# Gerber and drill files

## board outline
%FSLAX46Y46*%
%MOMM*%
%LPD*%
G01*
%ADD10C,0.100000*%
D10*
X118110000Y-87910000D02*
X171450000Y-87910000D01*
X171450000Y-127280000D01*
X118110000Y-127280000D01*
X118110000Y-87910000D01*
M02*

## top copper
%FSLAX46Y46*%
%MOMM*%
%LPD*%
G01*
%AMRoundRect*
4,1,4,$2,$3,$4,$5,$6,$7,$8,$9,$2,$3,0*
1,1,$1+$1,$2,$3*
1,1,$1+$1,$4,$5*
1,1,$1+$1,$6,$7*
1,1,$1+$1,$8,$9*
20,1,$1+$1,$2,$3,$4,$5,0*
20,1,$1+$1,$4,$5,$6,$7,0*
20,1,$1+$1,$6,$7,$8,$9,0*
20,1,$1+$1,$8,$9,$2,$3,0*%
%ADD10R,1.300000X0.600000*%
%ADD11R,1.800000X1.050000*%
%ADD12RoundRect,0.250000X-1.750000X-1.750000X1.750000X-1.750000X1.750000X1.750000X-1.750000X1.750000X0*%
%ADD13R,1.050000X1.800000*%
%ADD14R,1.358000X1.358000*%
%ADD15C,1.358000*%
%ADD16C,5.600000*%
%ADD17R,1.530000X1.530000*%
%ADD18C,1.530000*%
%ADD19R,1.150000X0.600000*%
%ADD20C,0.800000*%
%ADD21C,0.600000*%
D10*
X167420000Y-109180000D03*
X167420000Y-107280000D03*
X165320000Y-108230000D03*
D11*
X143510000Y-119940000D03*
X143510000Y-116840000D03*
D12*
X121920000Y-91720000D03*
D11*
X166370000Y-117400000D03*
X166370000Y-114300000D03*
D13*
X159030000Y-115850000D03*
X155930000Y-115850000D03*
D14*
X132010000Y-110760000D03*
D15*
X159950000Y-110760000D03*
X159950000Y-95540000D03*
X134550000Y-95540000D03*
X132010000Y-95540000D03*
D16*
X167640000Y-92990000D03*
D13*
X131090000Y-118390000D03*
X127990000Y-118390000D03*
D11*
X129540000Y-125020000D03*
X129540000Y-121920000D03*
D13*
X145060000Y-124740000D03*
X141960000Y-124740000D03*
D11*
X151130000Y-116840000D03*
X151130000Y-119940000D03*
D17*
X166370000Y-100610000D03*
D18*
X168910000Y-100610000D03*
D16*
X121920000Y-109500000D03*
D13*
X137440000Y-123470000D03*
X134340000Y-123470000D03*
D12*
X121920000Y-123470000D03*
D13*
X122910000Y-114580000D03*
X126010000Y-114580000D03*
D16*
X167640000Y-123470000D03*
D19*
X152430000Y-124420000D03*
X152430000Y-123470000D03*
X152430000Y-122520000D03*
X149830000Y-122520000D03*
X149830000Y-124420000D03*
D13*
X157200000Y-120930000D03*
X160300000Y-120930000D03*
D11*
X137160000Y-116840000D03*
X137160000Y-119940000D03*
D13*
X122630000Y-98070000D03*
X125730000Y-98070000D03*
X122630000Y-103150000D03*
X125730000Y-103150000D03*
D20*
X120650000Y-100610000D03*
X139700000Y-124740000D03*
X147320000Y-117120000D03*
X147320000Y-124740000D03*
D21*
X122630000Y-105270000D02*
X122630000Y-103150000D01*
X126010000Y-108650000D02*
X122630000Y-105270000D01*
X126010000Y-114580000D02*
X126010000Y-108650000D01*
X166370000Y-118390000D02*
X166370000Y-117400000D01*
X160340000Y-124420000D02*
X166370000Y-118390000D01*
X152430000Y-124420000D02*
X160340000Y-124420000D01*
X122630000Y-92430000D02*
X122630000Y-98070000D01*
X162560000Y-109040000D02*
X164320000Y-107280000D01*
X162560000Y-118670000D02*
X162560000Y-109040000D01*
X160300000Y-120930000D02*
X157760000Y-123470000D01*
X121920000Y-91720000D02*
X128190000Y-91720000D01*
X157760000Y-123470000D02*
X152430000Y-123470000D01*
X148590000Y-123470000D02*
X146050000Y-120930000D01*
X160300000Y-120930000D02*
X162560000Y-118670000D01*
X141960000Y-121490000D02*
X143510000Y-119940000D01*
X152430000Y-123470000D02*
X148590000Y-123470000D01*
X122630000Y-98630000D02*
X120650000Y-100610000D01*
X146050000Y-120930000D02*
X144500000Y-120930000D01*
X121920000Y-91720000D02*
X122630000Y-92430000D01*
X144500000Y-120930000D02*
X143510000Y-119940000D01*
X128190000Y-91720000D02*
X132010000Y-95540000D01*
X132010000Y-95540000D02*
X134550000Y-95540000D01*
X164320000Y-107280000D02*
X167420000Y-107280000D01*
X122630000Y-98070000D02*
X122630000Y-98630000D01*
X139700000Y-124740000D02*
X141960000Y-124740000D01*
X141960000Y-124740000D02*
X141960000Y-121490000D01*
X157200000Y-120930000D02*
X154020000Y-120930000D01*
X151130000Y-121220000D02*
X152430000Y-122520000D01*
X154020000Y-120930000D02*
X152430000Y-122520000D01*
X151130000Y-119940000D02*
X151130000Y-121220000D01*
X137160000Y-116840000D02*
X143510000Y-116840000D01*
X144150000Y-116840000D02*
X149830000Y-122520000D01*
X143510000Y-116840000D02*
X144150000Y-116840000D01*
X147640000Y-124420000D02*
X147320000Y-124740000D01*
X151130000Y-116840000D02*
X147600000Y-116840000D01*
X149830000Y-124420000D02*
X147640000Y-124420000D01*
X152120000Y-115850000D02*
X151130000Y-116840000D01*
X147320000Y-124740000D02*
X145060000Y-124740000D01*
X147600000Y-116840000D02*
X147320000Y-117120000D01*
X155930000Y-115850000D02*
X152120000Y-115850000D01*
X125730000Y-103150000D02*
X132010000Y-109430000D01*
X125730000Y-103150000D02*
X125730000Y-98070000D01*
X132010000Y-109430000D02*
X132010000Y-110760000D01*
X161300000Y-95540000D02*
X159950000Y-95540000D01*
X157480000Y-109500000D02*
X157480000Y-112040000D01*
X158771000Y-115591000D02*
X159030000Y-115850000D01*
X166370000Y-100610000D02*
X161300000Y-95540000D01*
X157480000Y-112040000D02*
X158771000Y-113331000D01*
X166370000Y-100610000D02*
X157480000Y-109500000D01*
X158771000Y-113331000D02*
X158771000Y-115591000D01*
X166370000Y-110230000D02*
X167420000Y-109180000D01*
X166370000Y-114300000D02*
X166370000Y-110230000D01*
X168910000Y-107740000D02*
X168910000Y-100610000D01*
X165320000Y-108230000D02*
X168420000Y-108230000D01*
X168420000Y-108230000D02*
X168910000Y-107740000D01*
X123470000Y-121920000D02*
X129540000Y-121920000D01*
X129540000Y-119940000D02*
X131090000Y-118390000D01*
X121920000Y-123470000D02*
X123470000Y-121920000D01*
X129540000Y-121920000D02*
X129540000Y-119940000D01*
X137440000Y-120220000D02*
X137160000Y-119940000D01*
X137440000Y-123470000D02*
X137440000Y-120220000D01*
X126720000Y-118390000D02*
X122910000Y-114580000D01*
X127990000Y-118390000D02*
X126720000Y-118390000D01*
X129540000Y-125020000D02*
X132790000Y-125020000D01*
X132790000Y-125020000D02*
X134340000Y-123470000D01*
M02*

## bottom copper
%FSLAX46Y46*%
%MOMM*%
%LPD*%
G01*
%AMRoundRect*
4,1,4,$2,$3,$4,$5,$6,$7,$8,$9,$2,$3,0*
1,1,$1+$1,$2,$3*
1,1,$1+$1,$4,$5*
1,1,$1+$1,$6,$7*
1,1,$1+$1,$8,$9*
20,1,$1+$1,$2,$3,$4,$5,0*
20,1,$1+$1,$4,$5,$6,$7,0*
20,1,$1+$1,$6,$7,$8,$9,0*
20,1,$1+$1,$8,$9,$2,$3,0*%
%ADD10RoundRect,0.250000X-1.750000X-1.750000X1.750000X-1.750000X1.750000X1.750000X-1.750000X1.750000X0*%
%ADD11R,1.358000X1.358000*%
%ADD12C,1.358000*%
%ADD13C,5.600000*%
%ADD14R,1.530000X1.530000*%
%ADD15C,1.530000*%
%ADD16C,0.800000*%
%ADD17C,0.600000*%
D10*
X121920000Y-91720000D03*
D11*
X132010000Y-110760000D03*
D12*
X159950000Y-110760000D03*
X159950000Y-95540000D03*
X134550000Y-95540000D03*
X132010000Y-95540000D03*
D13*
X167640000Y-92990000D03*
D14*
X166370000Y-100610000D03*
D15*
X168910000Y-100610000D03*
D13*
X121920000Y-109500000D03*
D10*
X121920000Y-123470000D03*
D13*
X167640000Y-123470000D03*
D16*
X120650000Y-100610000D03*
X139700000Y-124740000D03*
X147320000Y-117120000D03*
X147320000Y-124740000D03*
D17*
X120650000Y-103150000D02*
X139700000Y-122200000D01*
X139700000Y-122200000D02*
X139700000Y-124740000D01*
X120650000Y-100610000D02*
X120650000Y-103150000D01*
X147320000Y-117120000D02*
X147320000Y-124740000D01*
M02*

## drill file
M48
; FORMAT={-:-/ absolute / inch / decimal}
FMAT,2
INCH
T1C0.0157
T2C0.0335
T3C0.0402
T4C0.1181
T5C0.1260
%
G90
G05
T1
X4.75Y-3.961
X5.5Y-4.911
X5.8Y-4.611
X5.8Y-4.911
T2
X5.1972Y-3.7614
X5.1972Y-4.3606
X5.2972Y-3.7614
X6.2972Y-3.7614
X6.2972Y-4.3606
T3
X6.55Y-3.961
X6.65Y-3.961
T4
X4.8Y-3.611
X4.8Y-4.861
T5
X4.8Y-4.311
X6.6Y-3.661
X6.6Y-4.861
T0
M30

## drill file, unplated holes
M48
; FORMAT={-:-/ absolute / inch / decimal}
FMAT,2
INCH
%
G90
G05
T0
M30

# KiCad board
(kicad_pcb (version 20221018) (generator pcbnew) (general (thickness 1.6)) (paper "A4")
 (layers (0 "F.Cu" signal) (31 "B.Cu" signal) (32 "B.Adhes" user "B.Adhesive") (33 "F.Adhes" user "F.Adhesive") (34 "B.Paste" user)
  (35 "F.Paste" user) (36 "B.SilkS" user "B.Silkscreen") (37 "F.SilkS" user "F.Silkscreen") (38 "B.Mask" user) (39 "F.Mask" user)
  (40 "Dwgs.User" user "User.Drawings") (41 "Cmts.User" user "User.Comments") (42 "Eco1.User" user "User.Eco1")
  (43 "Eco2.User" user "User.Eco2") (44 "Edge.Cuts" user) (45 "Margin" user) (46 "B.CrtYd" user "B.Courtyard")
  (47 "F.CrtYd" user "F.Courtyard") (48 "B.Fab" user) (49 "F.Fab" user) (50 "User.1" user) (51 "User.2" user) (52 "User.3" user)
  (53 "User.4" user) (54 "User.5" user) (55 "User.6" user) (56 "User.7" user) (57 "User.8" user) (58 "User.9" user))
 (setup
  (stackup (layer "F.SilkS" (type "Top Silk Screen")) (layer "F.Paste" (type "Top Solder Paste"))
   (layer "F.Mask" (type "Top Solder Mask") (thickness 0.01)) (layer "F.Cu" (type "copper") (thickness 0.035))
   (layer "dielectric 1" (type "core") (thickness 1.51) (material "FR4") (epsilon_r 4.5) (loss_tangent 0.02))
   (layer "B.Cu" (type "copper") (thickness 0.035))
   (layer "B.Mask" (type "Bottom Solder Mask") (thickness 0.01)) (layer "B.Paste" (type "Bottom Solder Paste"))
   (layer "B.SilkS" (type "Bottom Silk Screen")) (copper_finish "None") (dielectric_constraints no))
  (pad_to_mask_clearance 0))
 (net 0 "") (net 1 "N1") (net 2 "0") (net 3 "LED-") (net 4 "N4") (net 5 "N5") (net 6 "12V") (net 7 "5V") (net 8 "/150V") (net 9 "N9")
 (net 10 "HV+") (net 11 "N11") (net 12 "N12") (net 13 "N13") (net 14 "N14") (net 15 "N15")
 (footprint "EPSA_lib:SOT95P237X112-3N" (layer "F.Cu") (at 166.37 108.23 180)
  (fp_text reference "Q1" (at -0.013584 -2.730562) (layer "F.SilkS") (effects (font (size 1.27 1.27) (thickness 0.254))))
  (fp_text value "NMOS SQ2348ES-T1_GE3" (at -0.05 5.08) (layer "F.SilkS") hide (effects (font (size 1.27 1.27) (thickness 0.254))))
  (pad "1" smd rect (at -1.05 -0.95 270) (size 0.6 1.3) (layers "F.Cu" "F.Paste" "F.Mask") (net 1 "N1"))
  (pad "2" smd rect (at -1.05 0.95 270) (size 0.6 1.3) (layers "F.Cu" "F.Paste" "F.Mask") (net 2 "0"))
  (pad "3" smd rect (at 1.05 0 270) (size 0.6 1.3) (layers "F.Cu" "F.Paste" "F.Mask") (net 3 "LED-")))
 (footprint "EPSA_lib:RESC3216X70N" (layer "F.Cu") (at 143.51 118.39 90)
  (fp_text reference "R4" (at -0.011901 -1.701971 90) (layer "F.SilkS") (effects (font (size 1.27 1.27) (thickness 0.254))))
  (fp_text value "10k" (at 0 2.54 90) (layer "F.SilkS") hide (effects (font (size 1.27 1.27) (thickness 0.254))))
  (pad "1" smd rect (at -1.55 0 90) (size 1.05 1.8) (layers "F.Cu" "F.Paste" "F.Mask") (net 2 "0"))
  (pad "2" smd rect (at 1.55 0 90) (size 1.05 1.8) (layers "F.Cu" "F.Paste" "F.Mask") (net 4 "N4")))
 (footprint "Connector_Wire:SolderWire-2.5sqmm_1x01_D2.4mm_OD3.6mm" (layer "F.Cu") (at 121.92 91.72)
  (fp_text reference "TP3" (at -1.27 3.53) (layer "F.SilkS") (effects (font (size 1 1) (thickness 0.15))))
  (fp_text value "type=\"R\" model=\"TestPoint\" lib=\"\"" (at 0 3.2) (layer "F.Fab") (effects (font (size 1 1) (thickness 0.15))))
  (pad "1" thru_hole roundrect (at 0 0) (size 4 4) (drill 3) (layers "*.Cu" "*.Mask") (roundrect_rratio 0.0625) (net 2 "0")))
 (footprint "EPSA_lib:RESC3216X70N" (layer "F.Cu") (at 166.37 115.85 90)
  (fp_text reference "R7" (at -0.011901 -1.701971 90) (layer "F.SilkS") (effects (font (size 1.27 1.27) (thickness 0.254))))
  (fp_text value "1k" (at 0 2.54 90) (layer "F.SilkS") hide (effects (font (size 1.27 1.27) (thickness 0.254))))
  (pad "1" smd rect (at -1.55 0 90) (size 1.05 1.8) (layers "F.Cu" "F.Paste" "F.Mask") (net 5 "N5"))
  (pad "2" smd rect (at 1.55 0 90) (size 1.05 1.8) (layers "F.Cu" "F.Paste" "F.Mask") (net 1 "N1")))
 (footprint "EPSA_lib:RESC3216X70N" (layer "F.Cu") (at 157.48 115.85 180)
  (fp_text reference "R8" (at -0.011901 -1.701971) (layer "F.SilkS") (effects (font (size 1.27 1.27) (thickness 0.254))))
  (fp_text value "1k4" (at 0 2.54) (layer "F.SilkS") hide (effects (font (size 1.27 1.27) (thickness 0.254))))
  (pad "1" smd rect (at -1.55 0 180) (size 1.05 1.8) (layers "F.Cu" "F.Paste" "F.Mask") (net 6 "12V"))
  (pad "2" smd rect (at 1.55 0 180) (size 1.05 1.8) (layers "F.Cu" "F.Paste" "F.Mask") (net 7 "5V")))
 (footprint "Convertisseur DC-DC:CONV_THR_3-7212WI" (layer "F.Cu") (at 146.05 103.15 180)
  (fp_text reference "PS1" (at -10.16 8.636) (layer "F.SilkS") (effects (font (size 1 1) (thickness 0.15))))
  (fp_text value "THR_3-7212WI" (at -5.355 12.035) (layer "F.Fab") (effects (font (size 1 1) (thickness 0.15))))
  (pad "1" thru_hole rect (at 14.04 -7.61 180) (size 1.358 1.358) (drill 0.85) (layers "*.Cu" "*.Mask") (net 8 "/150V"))
  (pad "12" thru_hole circle (at -13.9 -7.61 180) (size 1.358 1.358) (drill 0.85) (layers "*.Cu" "*.Mask") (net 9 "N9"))
  (pad "13" thru_hole circle (at -13.9 7.61 180) (size 1.358 1.358) (drill 0.85) (layers "*.Cu" "*.Mask") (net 6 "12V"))
  (pad "23" thru_hole circle (at 11.5 7.61 180) (size 1.358 1.358) (drill 0.85) (layers "*.Cu" "*.Mask") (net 2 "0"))
  (pad "24" thru_hole circle (at 14.04 7.61 180) (size 1.358 1.358) (drill 0.85) (layers "*.Cu" "*.Mask") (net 2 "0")))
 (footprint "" (layer "F.Cu") (at 167.64 92.99)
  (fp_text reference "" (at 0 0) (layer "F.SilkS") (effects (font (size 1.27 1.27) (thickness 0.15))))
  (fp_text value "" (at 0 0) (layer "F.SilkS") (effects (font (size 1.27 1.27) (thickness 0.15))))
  (pad "1" thru_hole circle (at 0 0) (size 5.6 5.6) (drill 3.2) (layers "*.Cu" "*.Mask")))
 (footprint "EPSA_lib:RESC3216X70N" (layer "F.Cu") (at 129.54 118.39 180)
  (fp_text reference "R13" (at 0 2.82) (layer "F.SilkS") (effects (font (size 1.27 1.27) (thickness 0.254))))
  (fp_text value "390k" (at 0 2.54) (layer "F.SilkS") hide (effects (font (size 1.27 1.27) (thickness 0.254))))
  (pad "1" smd rect (at -1.55 0 180) (size 1.05 1.8) (layers "F.Cu" "F.Paste" "F.Mask") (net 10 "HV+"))
  (pad "2" smd rect (at 1.55 0 180) (size 1.05 1.8) (layers "F.Cu" "F.Paste" "F.Mask") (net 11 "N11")))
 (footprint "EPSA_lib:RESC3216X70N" (layer "F.Cu") (at 129.54 123.47 90)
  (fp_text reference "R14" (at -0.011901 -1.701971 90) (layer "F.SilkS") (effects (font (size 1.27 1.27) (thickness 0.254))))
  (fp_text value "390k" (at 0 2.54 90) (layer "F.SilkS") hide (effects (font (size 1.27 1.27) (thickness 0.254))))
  (pad "1" smd rect (at -1.55 0 90) (size 1.05 1.8) (layers "F.Cu" "F.Paste" "F.Mask") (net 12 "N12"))
  (pad "2" smd rect (at 1.55 0 90) (size 1.05 1.8) (layers "F.Cu" "F.Paste" "F.Mask") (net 10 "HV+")))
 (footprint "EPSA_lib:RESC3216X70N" (layer "F.Cu") (at 143.51 124.74 180)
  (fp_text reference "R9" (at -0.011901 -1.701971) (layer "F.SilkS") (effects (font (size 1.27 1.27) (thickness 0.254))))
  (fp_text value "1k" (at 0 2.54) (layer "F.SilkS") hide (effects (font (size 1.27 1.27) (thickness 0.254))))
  (pad "1" smd rect (at -1.55 0 180) (size 1.05 1.8) (layers "F.Cu" "F.Paste" "F.Mask") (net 7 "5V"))
  (pad "2" smd rect (at 1.55 0 180) (size 1.05 1.8) (layers "F.Cu" "F.Paste" "F.Mask") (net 2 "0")))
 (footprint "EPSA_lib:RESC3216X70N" (layer "F.Cu") (at 151.13 118.39 -90)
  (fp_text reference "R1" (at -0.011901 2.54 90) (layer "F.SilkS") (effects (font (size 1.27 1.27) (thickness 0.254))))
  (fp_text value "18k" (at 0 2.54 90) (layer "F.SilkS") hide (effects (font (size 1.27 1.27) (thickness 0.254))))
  (pad "1" smd rect (at -1.55 0 270) (size 1.05 1.8) (layers "F.Cu" "F.Paste" "F.Mask") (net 7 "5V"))
  (pad "2" smd rect (at 1.55 0 270) (size 1.05 1.8) (layers "F.Cu" "F.Paste" "F.Mask") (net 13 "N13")))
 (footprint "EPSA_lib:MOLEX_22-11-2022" (layer "F.Cu") (at 166.37 100.61)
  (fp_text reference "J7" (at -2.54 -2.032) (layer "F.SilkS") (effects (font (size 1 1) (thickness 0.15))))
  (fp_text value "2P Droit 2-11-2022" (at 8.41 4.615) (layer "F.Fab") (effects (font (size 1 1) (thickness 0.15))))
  (pad "1" thru_hole rect (at 0 0) (size 1.53 1.53) (drill 1.02) (layers "*.Cu" "*.Mask") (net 6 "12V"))
  (pad "2" thru_hole circle (at 2.54 0) (size 1.53 1.53) (drill 1.02) (layers "*.Cu" "*.Mask") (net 3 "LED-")))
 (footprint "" (layer "F.Cu") (at 121.92 109.5)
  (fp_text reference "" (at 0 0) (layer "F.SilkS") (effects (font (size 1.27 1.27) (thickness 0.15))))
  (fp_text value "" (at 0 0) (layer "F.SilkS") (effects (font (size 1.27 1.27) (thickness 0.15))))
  (pad "1" thru_hole circle (at 0 0) (size 5.6 5.6) (drill 3.2) (layers "*.Cu" "*.Mask")))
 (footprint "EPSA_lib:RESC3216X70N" (layer "F.Cu") (at 135.89 123.47 180)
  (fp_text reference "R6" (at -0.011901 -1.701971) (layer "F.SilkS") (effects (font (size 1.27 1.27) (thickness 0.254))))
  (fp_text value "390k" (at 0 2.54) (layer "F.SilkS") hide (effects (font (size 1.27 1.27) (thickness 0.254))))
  (pad "1" smd rect (at -1.55 0 180) (size 1.05 1.8) (layers "F.Cu" "F.Paste" "F.Mask") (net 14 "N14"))
  (pad "2" smd rect (at 1.55 0 180) (size 1.05 1.8) (layers "F.Cu" "F.Paste" "F.Mask") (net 12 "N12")))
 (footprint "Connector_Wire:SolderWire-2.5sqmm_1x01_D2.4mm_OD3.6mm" (layer "F.Cu") (at 121.92 123.47)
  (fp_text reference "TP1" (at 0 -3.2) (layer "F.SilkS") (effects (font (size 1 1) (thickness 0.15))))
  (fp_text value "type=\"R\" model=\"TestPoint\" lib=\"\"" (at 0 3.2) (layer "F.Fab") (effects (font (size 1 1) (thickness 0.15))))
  (pad "1" thru_hole roundrect (at 0 0) (size 4 4) (drill 3) (layers "*.Cu" "*.Mask") (roundrect_rratio 0.0625) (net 10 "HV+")))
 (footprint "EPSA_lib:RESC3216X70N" (layer "F.Cu") (at 124.46 114.58)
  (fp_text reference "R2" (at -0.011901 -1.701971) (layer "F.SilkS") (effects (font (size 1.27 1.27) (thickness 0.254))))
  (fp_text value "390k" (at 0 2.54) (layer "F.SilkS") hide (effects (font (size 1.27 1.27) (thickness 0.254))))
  (pad "1" smd rect (at -1.55 0) (size 1.05 1.8) (layers "F.Cu" "F.Paste" "F.Mask") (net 11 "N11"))
  (pad "2" smd rect (at 1.55 0) (size 1.05 1.8) (layers "F.Cu" "F.Paste" "F.Mask") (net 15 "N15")))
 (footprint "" (layer "F.Cu") (at 167.64 123.47)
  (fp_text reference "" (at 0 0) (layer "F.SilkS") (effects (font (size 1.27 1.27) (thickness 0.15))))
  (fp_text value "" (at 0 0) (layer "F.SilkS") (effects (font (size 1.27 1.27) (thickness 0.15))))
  (pad "1" thru_hole circle (at 0 0) (size 5.6 5.6) (drill 3.2) (layers "*.Cu" "*.Mask")))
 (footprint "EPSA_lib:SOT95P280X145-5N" (layer "F.Cu") (at 151.13 123.47 180)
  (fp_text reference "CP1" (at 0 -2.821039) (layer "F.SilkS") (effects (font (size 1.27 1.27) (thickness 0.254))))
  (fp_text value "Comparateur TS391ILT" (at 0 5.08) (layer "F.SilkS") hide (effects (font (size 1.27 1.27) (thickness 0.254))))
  (pad "1" smd rect (at -1.3 -0.95 270) (size 0.6 1.15) (layers "F.Cu" "F.Paste" "F.Mask") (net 5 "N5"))
  (pad "2" smd rect (at -1.3 0 270) (size 0.6 1.15) (layers "F.Cu" "F.Paste" "F.Mask") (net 2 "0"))
  (pad "3" smd rect (at -1.3 0.95 270) (size 0.6 1.15) (layers "F.Cu" "F.Paste" "F.Mask") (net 13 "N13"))
  (pad "4" smd rect (at 1.3 0.95 270) (size 0.6 1.15) (layers "F.Cu" "F.Paste" "F.Mask") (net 4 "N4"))
  (pad "5" smd rect (at 1.3 -0.95 270) (size 0.6 1.15) (layers "F.Cu" "F.Paste" "F.Mask") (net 7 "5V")))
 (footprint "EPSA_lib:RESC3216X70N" (layer "F.Cu") (at 158.75 120.93)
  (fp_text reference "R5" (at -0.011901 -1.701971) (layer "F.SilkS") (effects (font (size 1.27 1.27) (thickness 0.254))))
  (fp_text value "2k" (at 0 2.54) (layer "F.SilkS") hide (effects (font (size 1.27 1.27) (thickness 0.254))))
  (pad "1" smd rect (at -1.55 0) (size 1.05 1.8) (layers "F.Cu" "F.Paste" "F.Mask") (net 13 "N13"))
  (pad "2" smd rect (at 1.55 0) (size 1.05 1.8) (layers "F.Cu" "F.Paste" "F.Mask") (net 2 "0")))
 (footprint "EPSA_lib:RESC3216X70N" (layer "F.Cu") (at 137.16 118.39 -90)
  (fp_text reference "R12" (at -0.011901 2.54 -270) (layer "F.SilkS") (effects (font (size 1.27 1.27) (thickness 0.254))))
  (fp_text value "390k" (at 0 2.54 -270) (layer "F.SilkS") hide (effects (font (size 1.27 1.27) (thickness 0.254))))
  (pad "1" smd rect (at -1.55 0 270) (size 1.05 1.8) (layers "F.Cu" "F.Paste" "F.Mask") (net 4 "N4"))
  (pad "2" smd rect (at 1.55 0 270) (size 1.05 1.8) (layers "F.Cu" "F.Paste" "F.Mask") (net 14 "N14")))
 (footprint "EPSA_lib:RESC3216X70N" (layer "F.Cu") (at 124.18 98.07)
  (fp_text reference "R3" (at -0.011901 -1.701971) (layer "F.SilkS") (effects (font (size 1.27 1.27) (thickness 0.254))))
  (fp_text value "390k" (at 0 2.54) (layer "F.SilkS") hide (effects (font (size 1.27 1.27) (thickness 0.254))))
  (pad "1" smd rect (at -1.55 0) (size 1.05 1.8) (layers "F.Cu" "F.Paste" "F.Mask") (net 2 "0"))
  (pad "2" smd rect (at 1.55 0) (size 1.05 1.8) (layers "F.Cu" "F.Paste" "F.Mask") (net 8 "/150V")))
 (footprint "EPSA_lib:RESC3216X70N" (layer "F.Cu") (at 124.18 103.15)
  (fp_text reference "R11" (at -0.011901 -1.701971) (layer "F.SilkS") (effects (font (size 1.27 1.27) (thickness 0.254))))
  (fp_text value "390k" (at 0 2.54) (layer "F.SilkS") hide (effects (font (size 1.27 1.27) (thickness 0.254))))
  (pad "1" smd rect (at -1.55 0) (size 1.05 1.8) (layers "F.Cu" "F.Paste" "F.Mask") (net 15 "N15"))
  (pad "2" smd rect (at 1.55 0) (size 1.05 1.8) (layers "F.Cu" "F.Paste" "F.Mask") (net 8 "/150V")))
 (gr_rect (start 118.11 87.91) (end 171.45 127.28) (stroke (width 0.1) (type default)) (fill none) (layer "Edge.Cuts"))
 (segment (start 166.37 118.39) (end 166.37 117.4) (width 0.6) (layer "F.Cu") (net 5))
 (segment (start 160.34 124.42) (end 166.37 118.39) (width 0.6) (layer "F.Cu") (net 5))
 (segment (start 152.43 124.42) (end 160.34 124.42) (width 0.6) (layer "F.Cu") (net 5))
 (segment (start 122.63 92.43) (end 122.63 98.07) (width 0.6) (layer "F.Cu") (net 2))
 (segment (start 162.56 109.04) (end 164.32 107.28) (width 0.6) (layer "F.Cu") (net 2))
 (segment (start 162.56 118.67) (end 162.56 109.04) (width 0.6) (layer "F.Cu") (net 2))
 (segment (start 160.3 120.93) (end 157.76 123.47) (width 0.6) (layer "F.Cu") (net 2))
 (segment (start 121.92 91.72) (end 128.19 91.72) (width 0.6) (layer "F.Cu") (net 2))
 (segment (start 157.76 123.47) (end 152.43 123.47) (width 0.6) (layer "F.Cu") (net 2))
 (segment (start 148.59 123.47) (end 146.05 120.93) (width 0.6) (layer "F.Cu") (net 2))
 (segment (start 160.3 120.93) (end 162.56 118.67) (width 0.6) (layer "F.Cu") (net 2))
 (segment (start 141.96 121.49) (end 143.51 119.94) (width 0.6) (layer "F.Cu") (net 2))
 (segment (start 152.43 123.47) (end 148.59 123.47) (width 0.6) (layer "F.Cu") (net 2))
 (segment (start 122.63 98.63) (end 120.65 100.61) (width 0.6) (layer "F.Cu") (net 2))
 (segment (start 146.05 120.93) (end 144.5 120.93) (width 0.6) (layer "F.Cu") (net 2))
 (segment (start 121.92 91.72) (end 122.63 92.43) (width 0.6) (layer "F.Cu") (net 2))
 (segment (start 144.5 120.93) (end 143.51 119.94) (width 0.6) (layer "F.Cu") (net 2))
 (segment (start 128.19 91.72) (end 132.01 95.54) (width 0.6) (layer "F.Cu") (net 2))
 (segment (start 132.01 95.54) (end 134.55 95.54) (width 0.6) (layer "F.Cu") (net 2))
 (segment (start 164.32 107.28) (end 167.42 107.28) (width 0.6) (layer "F.Cu") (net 2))
 (segment (start 122.63 98.07) (end 122.63 98.63) (width 0.6) (layer "F.Cu") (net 2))
 (segment (start 139.7 124.74) (end 141.96 124.74) (width 0.6) (layer "F.Cu") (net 2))
 (segment (start 141.96 124.74) (end 141.96 121.49) (width 0.6) (layer "F.Cu") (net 2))
 (via (at 120.65 100.61) (size 0.8) (drill 0.4) (layers "F.Cu" "B.Cu") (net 2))
 (via (at 139.7 124.74) (size 0.8) (drill 0.4) (layers "F.Cu" "B.Cu") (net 2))
 (segment (start 120.65 103.15) (end 139.7 122.2) (width 0.6) (layer "B.Cu") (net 2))
 (segment (start 139.7 122.2) (end 139.7 124.74) (width 0.6) (layer "B.Cu") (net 2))
 (segment (start 120.65 100.61) (end 120.65 103.15) (width 0.6) (layer "B.Cu") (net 2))
 (segment (start 157.2 120.93) (end 154.02 120.93) (width 0.6) (layer "F.Cu") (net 13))
 (segment (start 151.13 121.22) (end 152.43 122.52) (width 0.6) (layer "F.Cu") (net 13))
 (segment (start 154.02 120.93) (end 152.43 122.52) (width 0.6) (layer "F.Cu") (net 13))
 (segment (start 151.13 119.94) (end 151.13 121.22) (width 0.6) (layer "F.Cu") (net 13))
 (segment (start 137.16 116.84) (end 143.51 116.84) (width 0.6) (layer "F.Cu") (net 4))
 (segment (start 144.15 116.84) (end 149.83 122.52) (width 0.6) (layer "F.Cu") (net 4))
 (segment (start 143.51 116.84) (end 144.15 116.84) (width 0.6) (layer "F.Cu") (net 4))
 (segment (start 147.64 124.42) (end 147.32 124.74) (width 0.6) (layer "F.Cu") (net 7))
 (segment (start 151.13 116.84) (end 147.6 116.84) (width 0.6) (layer "F.Cu") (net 7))
 (segment (start 149.83 124.42) (end 147.64 124.42) (width 0.6) (layer "F.Cu") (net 7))
 (segment (start 152.12 115.85) (end 151.13 116.84) (width 0.6) (layer "F.Cu") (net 7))
 (segment (start 147.32 124.74) (end 145.06 124.74) (width 0.6) (layer "F.Cu") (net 7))
 (segment (start 147.6 116.84) (end 147.32 117.12) (width 0.6) (layer "F.Cu") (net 7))
 (segment (start 155.93 115.85) (end 152.12 115.85) (width 0.6) (layer "F.Cu") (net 7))
 (via (at 147.32 117.12) (size 0.8) (drill 0.4) (layers "F.Cu" "B.Cu") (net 7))
 (via (at 147.32 124.74) (size 0.8) (drill 0.4) (layers "F.Cu" "B.Cu") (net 7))
 (segment (start 147.32 117.12) (end 147.32 124.74) (width 0.6) (layer "B.Cu") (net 7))
 (segment (start 125.73 103.15) (end 132.01 109.43) (width 0.6) (layer "F.Cu") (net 8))
 (segment (start 125.73 103.15) (end 125.73 98.07) (width 0.6) (layer "F.Cu") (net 8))
 (segment (start 132.01 109.43) (end 132.01 110.76) (width 0.6) (layer "F.Cu") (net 8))
 (segment (start 161.3 95.54) (end 159.95 95.54) (width 0.6) (layer "F.Cu") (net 6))
 (segment (start 157.48 109.5) (end 157.48 112.04) (width 0.6) (layer "F.Cu") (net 6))
 (segment (start 158.771 115.591) (end 159.03 115.85) (width 0.6) (layer "F.Cu") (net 6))
 (segment (start 166.37 100.61) (end 161.3 95.54) (width 0.6) (layer "F.Cu") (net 6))
 (segment (start 157.48 112.04) (end 158.771 113.331) (width 0.6) (layer "F.Cu") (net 6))
 (segment (start 166.37 100.61) (end 157.48 109.5) (width 0.6) (layer "F.Cu") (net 6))
 (segment (start 158.771 113.331) (end 158.771 115.591) (width 0.6) (layer "F.Cu") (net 6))
 (segment (start 166.37 110.23) (end 167.42 109.18) (width 0.6) (layer "F.Cu") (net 1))
 (segment (start 166.37 114.3) (end 166.37 110.23) (width 0.6) (layer "F.Cu") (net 1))
 (segment (start 168.91 107.74) (end 168.91 100.61) (width 0.6) (layer "F.Cu") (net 3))
 (segment (start 165.32 108.23) (end 168.42 108.23) (width 0.6) (layer "F.Cu") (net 3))
 (segment (start 168.42 108.23) (end 168.91 107.74) (width 0.6) (layer "F.Cu") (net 3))
 (segment (start 123.47 121.92) (end 129.54 121.92) (width 0.6) (layer "F.Cu") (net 10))
 (segment (start 129.54 119.94) (end 131.09 118.39) (width 0.6) (layer "F.Cu") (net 10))
 (segment (start 121.92 123.47) (end 123.47 121.92) (width 0.6) (layer "F.Cu") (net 10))
 (segment (start 129.54 121.92) (end 129.54 119.94) (width 0.6) (layer "F.Cu") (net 10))
 (segment (start 126.01 114.58) (end 126.01 108.65) (width 0.6) (layer "F.Cu") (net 15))
 (segment (start 126.01 108.65) (end 122.63 105.27) (width 0.6) (layer "F.Cu") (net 15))
 (segment (start 122.63 105.27) (end 122.63 103.15) (width 0.6) (layer "F.Cu") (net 15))
 (segment (start 137.44 120.22) (end 137.16 119.94) (width 0.6) (layer "F.Cu") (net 14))
 (segment (start 137.44 123.47) (end 137.44 120.22) (width 0.6) (layer "F.Cu") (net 14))
 (segment (start 126.72 118.39) (end 122.91 114.58) (width 0.6) (layer "F.Cu") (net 11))
 (segment (start 127.99 118.39) (end 126.72 118.39) (width 0.6) (layer "F.Cu") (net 11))
 (segment (start 129.54 125.02) (end 132.79 125.02) (width 0.6) (layer "F.Cu") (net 12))
 (segment (start 132.79 125.02) (end 134.34 123.47) (width 0.6) (layer "F.Cu") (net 12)))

